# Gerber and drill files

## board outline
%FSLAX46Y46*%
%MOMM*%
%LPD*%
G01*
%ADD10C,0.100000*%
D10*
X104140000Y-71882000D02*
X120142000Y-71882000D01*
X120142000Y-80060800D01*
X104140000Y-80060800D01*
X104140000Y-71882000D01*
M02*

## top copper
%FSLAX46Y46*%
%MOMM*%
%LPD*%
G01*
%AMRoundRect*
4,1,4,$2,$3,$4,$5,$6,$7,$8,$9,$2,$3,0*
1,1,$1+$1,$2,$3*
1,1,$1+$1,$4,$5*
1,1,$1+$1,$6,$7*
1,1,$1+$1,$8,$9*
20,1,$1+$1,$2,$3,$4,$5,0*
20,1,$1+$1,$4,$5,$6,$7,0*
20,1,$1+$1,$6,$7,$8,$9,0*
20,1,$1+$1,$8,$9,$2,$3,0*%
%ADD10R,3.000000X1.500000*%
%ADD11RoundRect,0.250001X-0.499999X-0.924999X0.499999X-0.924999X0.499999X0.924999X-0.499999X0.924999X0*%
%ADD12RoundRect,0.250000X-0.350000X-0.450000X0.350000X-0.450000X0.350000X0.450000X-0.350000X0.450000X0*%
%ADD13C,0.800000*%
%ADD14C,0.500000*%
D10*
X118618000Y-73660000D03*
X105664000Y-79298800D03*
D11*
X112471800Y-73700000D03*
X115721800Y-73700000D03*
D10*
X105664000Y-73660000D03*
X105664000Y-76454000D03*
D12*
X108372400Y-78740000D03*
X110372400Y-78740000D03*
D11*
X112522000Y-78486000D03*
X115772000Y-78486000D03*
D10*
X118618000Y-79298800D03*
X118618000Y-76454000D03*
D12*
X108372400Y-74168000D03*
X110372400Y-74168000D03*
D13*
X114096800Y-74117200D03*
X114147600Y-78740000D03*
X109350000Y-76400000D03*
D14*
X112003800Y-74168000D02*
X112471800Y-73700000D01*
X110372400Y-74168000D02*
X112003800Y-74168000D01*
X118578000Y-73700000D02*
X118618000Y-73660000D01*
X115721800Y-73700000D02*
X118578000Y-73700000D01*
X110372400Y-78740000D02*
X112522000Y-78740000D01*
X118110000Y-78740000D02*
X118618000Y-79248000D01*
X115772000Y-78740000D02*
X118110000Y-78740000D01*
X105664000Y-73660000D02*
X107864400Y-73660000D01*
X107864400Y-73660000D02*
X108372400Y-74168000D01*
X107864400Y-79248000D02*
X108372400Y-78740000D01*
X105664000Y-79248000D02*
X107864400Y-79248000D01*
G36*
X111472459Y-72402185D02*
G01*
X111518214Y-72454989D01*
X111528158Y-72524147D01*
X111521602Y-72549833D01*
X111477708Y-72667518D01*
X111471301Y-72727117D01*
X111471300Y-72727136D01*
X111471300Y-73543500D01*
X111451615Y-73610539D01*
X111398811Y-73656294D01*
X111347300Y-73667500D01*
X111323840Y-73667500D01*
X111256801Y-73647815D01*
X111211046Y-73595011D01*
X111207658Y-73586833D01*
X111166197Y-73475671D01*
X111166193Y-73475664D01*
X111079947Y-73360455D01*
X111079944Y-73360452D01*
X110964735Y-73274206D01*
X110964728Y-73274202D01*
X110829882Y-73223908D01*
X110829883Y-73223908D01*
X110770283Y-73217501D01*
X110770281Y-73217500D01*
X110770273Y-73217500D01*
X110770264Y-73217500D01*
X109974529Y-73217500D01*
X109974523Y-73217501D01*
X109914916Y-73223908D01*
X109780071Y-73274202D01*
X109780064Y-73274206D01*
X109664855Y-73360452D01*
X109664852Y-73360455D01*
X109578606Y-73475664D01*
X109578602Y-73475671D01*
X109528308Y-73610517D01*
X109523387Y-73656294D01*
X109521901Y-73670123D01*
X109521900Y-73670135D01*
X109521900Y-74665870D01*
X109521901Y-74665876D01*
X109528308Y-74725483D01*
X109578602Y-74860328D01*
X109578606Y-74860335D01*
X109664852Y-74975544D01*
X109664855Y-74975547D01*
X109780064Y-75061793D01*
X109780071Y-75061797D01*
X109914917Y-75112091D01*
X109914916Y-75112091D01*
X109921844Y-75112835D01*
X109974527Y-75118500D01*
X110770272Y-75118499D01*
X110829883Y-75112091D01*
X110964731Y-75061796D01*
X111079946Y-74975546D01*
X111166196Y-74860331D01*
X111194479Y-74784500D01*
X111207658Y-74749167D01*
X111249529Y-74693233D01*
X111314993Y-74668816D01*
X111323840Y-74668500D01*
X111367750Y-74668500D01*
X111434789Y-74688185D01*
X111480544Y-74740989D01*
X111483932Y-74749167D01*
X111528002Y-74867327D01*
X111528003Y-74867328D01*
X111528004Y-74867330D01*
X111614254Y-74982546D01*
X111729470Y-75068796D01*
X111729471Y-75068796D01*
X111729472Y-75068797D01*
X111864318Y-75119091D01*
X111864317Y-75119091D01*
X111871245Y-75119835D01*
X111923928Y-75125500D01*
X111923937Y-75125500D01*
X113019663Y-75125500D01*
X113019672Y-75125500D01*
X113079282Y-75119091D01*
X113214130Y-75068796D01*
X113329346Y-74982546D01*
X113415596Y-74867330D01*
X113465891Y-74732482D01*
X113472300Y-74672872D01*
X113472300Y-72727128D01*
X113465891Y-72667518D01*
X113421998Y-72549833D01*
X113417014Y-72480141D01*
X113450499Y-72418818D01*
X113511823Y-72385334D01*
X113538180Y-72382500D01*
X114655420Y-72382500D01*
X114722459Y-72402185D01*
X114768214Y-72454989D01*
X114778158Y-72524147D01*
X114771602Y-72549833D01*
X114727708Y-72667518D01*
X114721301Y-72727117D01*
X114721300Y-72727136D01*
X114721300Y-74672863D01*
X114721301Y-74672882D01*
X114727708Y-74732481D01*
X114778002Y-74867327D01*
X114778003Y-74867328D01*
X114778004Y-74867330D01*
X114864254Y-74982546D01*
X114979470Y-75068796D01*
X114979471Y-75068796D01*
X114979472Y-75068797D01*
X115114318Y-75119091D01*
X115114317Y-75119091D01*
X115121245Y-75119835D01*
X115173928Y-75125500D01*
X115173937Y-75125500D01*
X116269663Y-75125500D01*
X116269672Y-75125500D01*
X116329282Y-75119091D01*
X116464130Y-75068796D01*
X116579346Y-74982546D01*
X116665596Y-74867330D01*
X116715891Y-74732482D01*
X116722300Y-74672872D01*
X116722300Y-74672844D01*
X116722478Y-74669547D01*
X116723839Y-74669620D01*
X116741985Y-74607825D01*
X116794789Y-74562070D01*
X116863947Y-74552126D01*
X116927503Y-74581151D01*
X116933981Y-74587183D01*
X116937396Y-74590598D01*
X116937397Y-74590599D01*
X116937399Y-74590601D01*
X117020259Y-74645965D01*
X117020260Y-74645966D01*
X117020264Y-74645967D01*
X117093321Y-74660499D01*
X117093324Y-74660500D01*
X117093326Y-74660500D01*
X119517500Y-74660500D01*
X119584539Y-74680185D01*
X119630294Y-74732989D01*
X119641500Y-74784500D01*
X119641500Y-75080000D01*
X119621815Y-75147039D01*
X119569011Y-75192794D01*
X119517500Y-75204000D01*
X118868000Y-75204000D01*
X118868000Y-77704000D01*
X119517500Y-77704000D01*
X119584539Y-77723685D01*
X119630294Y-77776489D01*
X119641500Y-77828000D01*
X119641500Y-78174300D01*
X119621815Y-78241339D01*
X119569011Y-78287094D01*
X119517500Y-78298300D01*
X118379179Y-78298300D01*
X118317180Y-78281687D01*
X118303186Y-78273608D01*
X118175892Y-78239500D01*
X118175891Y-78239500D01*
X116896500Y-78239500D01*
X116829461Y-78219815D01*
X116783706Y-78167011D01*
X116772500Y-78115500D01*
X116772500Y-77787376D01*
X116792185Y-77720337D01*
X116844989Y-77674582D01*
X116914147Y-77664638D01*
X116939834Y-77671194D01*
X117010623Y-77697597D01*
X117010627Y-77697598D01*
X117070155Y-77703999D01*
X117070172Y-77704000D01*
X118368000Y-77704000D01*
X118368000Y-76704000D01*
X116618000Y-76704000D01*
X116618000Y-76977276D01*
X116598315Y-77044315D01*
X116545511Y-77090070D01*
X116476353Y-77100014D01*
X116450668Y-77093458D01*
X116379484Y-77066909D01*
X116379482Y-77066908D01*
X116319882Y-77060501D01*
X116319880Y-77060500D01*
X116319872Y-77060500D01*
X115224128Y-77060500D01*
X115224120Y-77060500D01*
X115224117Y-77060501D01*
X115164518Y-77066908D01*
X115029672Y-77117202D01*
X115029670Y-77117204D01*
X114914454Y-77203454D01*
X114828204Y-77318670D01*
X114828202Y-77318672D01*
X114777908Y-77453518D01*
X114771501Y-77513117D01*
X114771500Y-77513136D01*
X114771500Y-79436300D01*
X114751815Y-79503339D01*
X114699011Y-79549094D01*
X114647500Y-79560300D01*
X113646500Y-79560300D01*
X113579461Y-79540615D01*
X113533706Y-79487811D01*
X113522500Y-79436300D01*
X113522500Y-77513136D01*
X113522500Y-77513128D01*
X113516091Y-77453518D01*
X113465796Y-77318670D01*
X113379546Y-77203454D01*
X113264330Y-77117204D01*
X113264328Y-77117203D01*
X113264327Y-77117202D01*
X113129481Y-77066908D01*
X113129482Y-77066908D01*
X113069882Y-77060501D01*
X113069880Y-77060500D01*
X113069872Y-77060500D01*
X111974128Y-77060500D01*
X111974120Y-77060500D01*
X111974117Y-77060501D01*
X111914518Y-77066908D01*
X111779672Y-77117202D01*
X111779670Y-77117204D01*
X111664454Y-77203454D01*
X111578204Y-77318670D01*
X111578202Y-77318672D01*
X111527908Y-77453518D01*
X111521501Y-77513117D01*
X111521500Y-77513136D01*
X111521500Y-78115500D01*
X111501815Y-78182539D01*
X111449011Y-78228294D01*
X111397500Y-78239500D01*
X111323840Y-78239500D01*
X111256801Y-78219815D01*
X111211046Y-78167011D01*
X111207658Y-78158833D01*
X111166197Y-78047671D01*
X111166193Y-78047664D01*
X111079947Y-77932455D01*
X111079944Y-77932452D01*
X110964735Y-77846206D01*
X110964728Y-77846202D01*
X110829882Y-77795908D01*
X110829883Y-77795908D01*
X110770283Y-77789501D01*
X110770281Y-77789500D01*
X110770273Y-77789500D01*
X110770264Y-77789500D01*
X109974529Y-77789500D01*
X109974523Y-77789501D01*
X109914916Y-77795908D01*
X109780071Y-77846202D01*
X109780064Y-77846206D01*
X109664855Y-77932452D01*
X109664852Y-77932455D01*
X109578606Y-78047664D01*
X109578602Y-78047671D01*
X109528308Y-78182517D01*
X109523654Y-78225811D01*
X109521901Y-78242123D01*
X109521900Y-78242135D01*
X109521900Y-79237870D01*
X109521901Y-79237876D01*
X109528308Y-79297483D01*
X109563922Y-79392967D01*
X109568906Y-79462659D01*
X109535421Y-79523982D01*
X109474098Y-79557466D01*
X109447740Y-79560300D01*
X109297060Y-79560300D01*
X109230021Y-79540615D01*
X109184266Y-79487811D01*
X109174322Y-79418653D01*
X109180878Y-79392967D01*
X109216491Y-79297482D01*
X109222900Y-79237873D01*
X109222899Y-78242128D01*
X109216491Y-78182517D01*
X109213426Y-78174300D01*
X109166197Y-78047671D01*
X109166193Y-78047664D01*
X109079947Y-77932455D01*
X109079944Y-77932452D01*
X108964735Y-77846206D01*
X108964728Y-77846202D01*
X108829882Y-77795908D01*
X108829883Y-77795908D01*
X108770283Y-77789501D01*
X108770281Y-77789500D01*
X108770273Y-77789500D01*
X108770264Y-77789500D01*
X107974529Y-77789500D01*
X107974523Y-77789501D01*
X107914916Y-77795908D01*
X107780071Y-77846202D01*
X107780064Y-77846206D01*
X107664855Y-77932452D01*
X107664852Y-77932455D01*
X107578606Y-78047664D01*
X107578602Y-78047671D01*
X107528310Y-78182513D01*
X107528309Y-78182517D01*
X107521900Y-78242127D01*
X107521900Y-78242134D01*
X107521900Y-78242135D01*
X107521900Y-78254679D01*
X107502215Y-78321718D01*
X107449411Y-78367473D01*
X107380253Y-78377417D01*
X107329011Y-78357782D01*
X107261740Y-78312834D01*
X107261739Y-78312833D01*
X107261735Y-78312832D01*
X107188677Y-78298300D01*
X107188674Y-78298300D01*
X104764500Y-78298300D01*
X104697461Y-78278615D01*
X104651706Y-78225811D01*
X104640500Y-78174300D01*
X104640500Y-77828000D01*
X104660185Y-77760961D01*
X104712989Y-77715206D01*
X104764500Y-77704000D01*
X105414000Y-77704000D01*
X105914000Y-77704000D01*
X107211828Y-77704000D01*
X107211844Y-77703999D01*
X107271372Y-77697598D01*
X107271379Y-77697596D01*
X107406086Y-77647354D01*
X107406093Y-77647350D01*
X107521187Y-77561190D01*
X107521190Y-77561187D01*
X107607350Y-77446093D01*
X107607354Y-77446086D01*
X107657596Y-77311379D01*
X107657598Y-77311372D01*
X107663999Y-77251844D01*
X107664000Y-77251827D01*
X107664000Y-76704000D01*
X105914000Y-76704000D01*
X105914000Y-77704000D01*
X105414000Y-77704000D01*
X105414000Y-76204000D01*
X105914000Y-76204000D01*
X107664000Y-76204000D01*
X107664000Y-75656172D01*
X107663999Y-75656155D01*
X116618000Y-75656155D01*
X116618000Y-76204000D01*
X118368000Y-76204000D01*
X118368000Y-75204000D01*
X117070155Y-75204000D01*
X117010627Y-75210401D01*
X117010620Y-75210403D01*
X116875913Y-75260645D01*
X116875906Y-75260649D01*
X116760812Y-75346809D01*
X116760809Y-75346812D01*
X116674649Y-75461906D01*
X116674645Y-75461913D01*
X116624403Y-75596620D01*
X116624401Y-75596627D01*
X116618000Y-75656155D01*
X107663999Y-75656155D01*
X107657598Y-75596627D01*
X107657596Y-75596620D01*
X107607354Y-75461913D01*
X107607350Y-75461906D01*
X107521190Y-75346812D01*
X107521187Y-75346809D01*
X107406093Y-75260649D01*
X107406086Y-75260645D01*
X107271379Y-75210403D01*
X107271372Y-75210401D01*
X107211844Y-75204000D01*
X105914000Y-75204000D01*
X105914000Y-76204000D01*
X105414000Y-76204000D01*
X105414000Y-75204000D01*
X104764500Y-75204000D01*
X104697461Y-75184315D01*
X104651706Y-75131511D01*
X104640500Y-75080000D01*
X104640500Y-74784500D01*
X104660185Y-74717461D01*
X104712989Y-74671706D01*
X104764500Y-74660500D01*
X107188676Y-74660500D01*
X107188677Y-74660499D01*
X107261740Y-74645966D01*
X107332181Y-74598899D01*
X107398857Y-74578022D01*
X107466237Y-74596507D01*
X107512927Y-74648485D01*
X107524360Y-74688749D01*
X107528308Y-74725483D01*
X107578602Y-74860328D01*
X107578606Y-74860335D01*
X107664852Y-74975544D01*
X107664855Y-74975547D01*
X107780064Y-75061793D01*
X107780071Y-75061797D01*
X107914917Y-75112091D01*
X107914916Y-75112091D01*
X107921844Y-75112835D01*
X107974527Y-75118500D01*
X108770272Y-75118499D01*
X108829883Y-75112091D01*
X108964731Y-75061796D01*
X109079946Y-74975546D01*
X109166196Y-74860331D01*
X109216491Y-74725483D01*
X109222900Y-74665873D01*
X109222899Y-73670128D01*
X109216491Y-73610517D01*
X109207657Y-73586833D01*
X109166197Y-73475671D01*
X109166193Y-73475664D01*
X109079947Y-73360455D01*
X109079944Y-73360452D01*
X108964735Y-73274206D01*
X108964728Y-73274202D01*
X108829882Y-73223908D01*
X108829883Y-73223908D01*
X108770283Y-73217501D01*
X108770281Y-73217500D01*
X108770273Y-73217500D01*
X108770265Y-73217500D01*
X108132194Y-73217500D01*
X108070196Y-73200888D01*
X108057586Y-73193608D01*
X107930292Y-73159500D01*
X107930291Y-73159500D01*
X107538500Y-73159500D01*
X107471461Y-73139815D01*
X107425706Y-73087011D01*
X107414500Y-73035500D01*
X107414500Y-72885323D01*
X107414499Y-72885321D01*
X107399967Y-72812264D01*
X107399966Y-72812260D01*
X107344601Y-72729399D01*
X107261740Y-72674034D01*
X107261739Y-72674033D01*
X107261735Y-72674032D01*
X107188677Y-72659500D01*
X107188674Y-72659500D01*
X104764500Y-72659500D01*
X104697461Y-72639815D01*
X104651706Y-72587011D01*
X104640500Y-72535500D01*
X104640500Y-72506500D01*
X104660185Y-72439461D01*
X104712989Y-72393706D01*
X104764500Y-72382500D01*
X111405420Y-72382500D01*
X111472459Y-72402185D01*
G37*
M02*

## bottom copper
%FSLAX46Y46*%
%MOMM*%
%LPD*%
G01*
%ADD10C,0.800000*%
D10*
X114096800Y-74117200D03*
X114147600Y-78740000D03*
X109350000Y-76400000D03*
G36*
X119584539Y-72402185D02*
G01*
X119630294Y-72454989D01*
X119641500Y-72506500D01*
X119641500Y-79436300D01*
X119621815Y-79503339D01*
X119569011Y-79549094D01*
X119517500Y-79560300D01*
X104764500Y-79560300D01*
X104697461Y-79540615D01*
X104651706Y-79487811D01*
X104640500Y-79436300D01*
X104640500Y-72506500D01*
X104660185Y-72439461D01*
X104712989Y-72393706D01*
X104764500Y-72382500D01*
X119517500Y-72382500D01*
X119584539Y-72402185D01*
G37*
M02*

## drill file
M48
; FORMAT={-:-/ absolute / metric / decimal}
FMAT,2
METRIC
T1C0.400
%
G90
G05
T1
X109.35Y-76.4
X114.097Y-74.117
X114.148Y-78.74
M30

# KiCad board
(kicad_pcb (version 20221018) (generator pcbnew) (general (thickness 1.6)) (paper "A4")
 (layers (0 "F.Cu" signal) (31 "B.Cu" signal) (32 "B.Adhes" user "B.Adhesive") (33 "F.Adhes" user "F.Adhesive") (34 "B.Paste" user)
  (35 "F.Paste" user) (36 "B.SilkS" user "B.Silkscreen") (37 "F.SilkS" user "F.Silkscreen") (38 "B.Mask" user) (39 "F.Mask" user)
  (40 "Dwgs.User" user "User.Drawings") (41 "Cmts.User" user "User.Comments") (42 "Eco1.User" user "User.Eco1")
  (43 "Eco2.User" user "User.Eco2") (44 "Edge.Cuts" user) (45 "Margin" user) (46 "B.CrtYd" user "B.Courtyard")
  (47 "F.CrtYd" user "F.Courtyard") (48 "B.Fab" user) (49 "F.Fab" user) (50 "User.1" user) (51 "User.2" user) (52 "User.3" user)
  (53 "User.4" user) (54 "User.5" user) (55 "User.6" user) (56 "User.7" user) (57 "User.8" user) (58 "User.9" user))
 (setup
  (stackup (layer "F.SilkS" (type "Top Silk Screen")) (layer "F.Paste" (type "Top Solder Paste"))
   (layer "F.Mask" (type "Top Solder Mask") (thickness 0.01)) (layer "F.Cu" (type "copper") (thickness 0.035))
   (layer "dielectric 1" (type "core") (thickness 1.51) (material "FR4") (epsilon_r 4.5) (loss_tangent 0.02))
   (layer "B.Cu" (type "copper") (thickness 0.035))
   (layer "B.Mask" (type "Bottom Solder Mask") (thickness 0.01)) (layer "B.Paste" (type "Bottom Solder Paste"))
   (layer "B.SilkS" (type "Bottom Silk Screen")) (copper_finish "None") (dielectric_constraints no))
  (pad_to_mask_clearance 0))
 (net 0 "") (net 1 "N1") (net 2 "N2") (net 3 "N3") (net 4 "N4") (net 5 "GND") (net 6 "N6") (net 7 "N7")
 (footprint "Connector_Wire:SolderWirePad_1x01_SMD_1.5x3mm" (layer "F.Cu") (at 118.618 73.66 90)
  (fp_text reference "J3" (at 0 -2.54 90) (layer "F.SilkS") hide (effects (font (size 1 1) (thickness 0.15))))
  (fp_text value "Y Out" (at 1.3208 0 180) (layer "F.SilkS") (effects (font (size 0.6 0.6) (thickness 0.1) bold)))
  (pad "1" smd rect (at 0 0 90) (size 1.5 3) (layers "F.Cu" "F.Paste" "F.Mask") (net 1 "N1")))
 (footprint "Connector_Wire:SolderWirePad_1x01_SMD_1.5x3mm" (layer "F.Cu") (at 105.664 79.2988 -90)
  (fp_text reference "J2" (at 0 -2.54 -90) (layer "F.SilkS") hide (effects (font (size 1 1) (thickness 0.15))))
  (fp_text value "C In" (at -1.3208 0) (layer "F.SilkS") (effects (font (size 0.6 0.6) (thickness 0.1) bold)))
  (pad "1" smd rect (at 0 0 270) (size 1.5 3) (layers "F.Cu" "F.Paste" "F.Mask") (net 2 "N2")))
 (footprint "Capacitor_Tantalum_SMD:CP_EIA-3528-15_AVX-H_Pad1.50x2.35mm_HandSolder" (layer "F.Cu") (at 114.0968 73.7)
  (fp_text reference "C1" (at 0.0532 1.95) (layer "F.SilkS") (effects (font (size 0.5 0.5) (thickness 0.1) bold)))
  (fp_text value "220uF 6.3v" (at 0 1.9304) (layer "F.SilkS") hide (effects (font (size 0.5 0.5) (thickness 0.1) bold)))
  (pad "1" smd roundrect (at -1.625 0) (size 1.5 2.35) (layers "F.Cu" "F.Paste" "F.Mask") (roundrect_rratio 0.1666673333) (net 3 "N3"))
  (pad "2" smd roundrect (at 1.625 0) (size 1.5 2.35) (layers "F.Cu" "F.Paste" "F.Mask") (roundrect_rratio 0.1666673333) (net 1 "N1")))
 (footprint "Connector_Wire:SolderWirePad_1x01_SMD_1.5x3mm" (layer "F.Cu") (at 105.664 73.66 -90)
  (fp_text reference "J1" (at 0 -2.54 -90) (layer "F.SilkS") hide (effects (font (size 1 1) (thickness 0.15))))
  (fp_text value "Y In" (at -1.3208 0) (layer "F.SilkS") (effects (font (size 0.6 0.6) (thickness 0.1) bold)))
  (pad "1" smd rect (at 0 0 270) (size 1.5 3) (layers "F.Cu" "F.Paste" "F.Mask") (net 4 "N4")))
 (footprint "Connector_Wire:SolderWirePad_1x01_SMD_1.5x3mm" (layer "F.Cu") (at 105.664 76.454 90)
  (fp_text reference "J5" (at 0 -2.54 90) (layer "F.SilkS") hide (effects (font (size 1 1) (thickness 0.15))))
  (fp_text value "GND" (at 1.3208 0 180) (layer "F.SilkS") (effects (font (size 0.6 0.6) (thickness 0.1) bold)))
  (pad "1" smd rect (at 0 0 90) (size 1.5 3) (layers "F.Cu" "F.Paste" "F.Mask") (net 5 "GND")))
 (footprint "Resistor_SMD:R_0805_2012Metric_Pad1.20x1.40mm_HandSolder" (layer "F.Cu") (at 109.3724 78.74)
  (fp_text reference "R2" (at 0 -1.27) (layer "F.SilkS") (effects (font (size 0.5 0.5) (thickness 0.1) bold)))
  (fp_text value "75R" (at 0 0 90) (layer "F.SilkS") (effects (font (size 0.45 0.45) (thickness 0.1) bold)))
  (pad "1" smd roundrect (at -1 0) (size 1.2 1.4) (layers "F.Cu" "F.Paste" "F.Mask") (roundrect_rratio 0.2083333333) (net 2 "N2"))
  (pad "2" smd roundrect (at 1 0) (size 1.2 1.4) (layers "F.Cu" "F.Paste" "F.Mask") (roundrect_rratio 0.2083333333) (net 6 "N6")))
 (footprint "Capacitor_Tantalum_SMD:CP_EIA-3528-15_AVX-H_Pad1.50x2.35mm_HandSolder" (layer "F.Cu") (at 114.147 78.486)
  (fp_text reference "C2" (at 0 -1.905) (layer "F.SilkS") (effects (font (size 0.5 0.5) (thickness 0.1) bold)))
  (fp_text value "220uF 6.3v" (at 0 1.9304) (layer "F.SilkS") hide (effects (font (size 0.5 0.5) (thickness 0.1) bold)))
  (pad "1" smd roundrect (at -1.625 0) (size 1.5 2.35) (layers "F.Cu" "F.Paste" "F.Mask") (roundrect_rratio 0.1666673333) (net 6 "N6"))
  (pad "2" smd roundrect (at 1.625 0) (size 1.5 2.35) (layers "F.Cu" "F.Paste" "F.Mask") (roundrect_rratio 0.1666673333) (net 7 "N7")))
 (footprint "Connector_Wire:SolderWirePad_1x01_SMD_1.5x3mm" (layer "F.Cu") (at 118.618 79.2988 90)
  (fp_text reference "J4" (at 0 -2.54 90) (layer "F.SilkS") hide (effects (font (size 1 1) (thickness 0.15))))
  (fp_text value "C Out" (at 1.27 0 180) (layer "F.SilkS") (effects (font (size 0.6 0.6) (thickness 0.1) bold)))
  (pad "1" smd rect (at 0 0 90) (size 1.5 3) (layers "F.Cu" "F.Paste" "F.Mask") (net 7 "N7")))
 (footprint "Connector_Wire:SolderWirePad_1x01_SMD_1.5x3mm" (layer "F.Cu") (at 118.618 76.454 90)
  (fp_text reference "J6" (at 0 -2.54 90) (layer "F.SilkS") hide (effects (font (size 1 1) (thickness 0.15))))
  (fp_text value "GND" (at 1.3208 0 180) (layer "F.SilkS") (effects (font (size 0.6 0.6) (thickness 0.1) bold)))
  (pad "1" smd rect (at 0 0 90) (size 1.5 3) (layers "F.Cu" "F.Paste" "F.Mask") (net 5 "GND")))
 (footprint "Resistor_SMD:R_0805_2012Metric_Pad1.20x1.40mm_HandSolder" (layer "F.Cu") (at 109.3724 74.168)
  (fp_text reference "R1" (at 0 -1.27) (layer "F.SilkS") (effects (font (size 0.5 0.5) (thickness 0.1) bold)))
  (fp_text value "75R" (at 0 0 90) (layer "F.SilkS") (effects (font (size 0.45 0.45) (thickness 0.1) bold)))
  (pad "1" smd roundrect (at -1 0) (size 1.2 1.4) (layers "F.Cu" "F.Paste" "F.Mask") (roundrect_rratio 0.2083333333) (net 4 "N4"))
  (pad "2" smd roundrect (at 1 0) (size 1.2 1.4) (layers "F.Cu" "F.Paste" "F.Mask") (roundrect_rratio 0.2083333333) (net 3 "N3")))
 (gr_rect (start 104.14 71.882) (end 120.142 80.0608) (stroke (width 0.1) (type default)) (fill none) (layer "Edge.Cuts"))
 (segment (start 112.0038 74.168) (end 112.4718 73.7) (width 0.5) (layer "F.Cu") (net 3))
 (segment (start 110.3724 74.168) (end 112.0038 74.168) (width 0.5) (layer "F.Cu") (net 3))
 (segment (start 118.578 73.7) (end 118.618 73.66) (width 0.5) (layer "F.Cu") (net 1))
 (segment (start 115.7218 73.7) (end 118.578 73.7) (width 0.5) (layer "F.Cu") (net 1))
 (segment (start 110.3724 78.74) (end 112.522 78.74) (width 0.5) (layer "F.Cu") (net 6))
 (segment (start 118.11 78.74) (end 118.618 79.248) (width 0.5) (layer "F.Cu") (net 7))
 (segment (start 115.772 78.74) (end 118.11 78.74) (width 0.5) (layer "F.Cu") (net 7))
 (segment (start 105.664 73.66) (end 107.8644 73.66) (width 0.5) (layer "F.Cu") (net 4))
 (segment (start 107.8644 73.66) (end 108.3724 74.168) (width 0.5) (layer "F.Cu") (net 4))
 (segment (start 107.8644 79.248) (end 108.3724 78.74) (width 0.5) (layer "F.Cu") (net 2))
 (segment (start 105.664 79.248) (end 107.8644 79.248) (width 0.5) (layer "F.Cu") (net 2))
 (via (at 114.0968 74.1172) (size 0.8) (drill 0.4) (layers "F.Cu" "B.Cu") (free) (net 5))
 (via (at 114.1476 78.74) (size 0.8) (drill 0.4) (layers "F.Cu" "B.Cu") (free) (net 5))
 (via (at 109.35 76.4) (size 0.8) (drill 0.4) (layers "F.Cu" "B.Cu") (free) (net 5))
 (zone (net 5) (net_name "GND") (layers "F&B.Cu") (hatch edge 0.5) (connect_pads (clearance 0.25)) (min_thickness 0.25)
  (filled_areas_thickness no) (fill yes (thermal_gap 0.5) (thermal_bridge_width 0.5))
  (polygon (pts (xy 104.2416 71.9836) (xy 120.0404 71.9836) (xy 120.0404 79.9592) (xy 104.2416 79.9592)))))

